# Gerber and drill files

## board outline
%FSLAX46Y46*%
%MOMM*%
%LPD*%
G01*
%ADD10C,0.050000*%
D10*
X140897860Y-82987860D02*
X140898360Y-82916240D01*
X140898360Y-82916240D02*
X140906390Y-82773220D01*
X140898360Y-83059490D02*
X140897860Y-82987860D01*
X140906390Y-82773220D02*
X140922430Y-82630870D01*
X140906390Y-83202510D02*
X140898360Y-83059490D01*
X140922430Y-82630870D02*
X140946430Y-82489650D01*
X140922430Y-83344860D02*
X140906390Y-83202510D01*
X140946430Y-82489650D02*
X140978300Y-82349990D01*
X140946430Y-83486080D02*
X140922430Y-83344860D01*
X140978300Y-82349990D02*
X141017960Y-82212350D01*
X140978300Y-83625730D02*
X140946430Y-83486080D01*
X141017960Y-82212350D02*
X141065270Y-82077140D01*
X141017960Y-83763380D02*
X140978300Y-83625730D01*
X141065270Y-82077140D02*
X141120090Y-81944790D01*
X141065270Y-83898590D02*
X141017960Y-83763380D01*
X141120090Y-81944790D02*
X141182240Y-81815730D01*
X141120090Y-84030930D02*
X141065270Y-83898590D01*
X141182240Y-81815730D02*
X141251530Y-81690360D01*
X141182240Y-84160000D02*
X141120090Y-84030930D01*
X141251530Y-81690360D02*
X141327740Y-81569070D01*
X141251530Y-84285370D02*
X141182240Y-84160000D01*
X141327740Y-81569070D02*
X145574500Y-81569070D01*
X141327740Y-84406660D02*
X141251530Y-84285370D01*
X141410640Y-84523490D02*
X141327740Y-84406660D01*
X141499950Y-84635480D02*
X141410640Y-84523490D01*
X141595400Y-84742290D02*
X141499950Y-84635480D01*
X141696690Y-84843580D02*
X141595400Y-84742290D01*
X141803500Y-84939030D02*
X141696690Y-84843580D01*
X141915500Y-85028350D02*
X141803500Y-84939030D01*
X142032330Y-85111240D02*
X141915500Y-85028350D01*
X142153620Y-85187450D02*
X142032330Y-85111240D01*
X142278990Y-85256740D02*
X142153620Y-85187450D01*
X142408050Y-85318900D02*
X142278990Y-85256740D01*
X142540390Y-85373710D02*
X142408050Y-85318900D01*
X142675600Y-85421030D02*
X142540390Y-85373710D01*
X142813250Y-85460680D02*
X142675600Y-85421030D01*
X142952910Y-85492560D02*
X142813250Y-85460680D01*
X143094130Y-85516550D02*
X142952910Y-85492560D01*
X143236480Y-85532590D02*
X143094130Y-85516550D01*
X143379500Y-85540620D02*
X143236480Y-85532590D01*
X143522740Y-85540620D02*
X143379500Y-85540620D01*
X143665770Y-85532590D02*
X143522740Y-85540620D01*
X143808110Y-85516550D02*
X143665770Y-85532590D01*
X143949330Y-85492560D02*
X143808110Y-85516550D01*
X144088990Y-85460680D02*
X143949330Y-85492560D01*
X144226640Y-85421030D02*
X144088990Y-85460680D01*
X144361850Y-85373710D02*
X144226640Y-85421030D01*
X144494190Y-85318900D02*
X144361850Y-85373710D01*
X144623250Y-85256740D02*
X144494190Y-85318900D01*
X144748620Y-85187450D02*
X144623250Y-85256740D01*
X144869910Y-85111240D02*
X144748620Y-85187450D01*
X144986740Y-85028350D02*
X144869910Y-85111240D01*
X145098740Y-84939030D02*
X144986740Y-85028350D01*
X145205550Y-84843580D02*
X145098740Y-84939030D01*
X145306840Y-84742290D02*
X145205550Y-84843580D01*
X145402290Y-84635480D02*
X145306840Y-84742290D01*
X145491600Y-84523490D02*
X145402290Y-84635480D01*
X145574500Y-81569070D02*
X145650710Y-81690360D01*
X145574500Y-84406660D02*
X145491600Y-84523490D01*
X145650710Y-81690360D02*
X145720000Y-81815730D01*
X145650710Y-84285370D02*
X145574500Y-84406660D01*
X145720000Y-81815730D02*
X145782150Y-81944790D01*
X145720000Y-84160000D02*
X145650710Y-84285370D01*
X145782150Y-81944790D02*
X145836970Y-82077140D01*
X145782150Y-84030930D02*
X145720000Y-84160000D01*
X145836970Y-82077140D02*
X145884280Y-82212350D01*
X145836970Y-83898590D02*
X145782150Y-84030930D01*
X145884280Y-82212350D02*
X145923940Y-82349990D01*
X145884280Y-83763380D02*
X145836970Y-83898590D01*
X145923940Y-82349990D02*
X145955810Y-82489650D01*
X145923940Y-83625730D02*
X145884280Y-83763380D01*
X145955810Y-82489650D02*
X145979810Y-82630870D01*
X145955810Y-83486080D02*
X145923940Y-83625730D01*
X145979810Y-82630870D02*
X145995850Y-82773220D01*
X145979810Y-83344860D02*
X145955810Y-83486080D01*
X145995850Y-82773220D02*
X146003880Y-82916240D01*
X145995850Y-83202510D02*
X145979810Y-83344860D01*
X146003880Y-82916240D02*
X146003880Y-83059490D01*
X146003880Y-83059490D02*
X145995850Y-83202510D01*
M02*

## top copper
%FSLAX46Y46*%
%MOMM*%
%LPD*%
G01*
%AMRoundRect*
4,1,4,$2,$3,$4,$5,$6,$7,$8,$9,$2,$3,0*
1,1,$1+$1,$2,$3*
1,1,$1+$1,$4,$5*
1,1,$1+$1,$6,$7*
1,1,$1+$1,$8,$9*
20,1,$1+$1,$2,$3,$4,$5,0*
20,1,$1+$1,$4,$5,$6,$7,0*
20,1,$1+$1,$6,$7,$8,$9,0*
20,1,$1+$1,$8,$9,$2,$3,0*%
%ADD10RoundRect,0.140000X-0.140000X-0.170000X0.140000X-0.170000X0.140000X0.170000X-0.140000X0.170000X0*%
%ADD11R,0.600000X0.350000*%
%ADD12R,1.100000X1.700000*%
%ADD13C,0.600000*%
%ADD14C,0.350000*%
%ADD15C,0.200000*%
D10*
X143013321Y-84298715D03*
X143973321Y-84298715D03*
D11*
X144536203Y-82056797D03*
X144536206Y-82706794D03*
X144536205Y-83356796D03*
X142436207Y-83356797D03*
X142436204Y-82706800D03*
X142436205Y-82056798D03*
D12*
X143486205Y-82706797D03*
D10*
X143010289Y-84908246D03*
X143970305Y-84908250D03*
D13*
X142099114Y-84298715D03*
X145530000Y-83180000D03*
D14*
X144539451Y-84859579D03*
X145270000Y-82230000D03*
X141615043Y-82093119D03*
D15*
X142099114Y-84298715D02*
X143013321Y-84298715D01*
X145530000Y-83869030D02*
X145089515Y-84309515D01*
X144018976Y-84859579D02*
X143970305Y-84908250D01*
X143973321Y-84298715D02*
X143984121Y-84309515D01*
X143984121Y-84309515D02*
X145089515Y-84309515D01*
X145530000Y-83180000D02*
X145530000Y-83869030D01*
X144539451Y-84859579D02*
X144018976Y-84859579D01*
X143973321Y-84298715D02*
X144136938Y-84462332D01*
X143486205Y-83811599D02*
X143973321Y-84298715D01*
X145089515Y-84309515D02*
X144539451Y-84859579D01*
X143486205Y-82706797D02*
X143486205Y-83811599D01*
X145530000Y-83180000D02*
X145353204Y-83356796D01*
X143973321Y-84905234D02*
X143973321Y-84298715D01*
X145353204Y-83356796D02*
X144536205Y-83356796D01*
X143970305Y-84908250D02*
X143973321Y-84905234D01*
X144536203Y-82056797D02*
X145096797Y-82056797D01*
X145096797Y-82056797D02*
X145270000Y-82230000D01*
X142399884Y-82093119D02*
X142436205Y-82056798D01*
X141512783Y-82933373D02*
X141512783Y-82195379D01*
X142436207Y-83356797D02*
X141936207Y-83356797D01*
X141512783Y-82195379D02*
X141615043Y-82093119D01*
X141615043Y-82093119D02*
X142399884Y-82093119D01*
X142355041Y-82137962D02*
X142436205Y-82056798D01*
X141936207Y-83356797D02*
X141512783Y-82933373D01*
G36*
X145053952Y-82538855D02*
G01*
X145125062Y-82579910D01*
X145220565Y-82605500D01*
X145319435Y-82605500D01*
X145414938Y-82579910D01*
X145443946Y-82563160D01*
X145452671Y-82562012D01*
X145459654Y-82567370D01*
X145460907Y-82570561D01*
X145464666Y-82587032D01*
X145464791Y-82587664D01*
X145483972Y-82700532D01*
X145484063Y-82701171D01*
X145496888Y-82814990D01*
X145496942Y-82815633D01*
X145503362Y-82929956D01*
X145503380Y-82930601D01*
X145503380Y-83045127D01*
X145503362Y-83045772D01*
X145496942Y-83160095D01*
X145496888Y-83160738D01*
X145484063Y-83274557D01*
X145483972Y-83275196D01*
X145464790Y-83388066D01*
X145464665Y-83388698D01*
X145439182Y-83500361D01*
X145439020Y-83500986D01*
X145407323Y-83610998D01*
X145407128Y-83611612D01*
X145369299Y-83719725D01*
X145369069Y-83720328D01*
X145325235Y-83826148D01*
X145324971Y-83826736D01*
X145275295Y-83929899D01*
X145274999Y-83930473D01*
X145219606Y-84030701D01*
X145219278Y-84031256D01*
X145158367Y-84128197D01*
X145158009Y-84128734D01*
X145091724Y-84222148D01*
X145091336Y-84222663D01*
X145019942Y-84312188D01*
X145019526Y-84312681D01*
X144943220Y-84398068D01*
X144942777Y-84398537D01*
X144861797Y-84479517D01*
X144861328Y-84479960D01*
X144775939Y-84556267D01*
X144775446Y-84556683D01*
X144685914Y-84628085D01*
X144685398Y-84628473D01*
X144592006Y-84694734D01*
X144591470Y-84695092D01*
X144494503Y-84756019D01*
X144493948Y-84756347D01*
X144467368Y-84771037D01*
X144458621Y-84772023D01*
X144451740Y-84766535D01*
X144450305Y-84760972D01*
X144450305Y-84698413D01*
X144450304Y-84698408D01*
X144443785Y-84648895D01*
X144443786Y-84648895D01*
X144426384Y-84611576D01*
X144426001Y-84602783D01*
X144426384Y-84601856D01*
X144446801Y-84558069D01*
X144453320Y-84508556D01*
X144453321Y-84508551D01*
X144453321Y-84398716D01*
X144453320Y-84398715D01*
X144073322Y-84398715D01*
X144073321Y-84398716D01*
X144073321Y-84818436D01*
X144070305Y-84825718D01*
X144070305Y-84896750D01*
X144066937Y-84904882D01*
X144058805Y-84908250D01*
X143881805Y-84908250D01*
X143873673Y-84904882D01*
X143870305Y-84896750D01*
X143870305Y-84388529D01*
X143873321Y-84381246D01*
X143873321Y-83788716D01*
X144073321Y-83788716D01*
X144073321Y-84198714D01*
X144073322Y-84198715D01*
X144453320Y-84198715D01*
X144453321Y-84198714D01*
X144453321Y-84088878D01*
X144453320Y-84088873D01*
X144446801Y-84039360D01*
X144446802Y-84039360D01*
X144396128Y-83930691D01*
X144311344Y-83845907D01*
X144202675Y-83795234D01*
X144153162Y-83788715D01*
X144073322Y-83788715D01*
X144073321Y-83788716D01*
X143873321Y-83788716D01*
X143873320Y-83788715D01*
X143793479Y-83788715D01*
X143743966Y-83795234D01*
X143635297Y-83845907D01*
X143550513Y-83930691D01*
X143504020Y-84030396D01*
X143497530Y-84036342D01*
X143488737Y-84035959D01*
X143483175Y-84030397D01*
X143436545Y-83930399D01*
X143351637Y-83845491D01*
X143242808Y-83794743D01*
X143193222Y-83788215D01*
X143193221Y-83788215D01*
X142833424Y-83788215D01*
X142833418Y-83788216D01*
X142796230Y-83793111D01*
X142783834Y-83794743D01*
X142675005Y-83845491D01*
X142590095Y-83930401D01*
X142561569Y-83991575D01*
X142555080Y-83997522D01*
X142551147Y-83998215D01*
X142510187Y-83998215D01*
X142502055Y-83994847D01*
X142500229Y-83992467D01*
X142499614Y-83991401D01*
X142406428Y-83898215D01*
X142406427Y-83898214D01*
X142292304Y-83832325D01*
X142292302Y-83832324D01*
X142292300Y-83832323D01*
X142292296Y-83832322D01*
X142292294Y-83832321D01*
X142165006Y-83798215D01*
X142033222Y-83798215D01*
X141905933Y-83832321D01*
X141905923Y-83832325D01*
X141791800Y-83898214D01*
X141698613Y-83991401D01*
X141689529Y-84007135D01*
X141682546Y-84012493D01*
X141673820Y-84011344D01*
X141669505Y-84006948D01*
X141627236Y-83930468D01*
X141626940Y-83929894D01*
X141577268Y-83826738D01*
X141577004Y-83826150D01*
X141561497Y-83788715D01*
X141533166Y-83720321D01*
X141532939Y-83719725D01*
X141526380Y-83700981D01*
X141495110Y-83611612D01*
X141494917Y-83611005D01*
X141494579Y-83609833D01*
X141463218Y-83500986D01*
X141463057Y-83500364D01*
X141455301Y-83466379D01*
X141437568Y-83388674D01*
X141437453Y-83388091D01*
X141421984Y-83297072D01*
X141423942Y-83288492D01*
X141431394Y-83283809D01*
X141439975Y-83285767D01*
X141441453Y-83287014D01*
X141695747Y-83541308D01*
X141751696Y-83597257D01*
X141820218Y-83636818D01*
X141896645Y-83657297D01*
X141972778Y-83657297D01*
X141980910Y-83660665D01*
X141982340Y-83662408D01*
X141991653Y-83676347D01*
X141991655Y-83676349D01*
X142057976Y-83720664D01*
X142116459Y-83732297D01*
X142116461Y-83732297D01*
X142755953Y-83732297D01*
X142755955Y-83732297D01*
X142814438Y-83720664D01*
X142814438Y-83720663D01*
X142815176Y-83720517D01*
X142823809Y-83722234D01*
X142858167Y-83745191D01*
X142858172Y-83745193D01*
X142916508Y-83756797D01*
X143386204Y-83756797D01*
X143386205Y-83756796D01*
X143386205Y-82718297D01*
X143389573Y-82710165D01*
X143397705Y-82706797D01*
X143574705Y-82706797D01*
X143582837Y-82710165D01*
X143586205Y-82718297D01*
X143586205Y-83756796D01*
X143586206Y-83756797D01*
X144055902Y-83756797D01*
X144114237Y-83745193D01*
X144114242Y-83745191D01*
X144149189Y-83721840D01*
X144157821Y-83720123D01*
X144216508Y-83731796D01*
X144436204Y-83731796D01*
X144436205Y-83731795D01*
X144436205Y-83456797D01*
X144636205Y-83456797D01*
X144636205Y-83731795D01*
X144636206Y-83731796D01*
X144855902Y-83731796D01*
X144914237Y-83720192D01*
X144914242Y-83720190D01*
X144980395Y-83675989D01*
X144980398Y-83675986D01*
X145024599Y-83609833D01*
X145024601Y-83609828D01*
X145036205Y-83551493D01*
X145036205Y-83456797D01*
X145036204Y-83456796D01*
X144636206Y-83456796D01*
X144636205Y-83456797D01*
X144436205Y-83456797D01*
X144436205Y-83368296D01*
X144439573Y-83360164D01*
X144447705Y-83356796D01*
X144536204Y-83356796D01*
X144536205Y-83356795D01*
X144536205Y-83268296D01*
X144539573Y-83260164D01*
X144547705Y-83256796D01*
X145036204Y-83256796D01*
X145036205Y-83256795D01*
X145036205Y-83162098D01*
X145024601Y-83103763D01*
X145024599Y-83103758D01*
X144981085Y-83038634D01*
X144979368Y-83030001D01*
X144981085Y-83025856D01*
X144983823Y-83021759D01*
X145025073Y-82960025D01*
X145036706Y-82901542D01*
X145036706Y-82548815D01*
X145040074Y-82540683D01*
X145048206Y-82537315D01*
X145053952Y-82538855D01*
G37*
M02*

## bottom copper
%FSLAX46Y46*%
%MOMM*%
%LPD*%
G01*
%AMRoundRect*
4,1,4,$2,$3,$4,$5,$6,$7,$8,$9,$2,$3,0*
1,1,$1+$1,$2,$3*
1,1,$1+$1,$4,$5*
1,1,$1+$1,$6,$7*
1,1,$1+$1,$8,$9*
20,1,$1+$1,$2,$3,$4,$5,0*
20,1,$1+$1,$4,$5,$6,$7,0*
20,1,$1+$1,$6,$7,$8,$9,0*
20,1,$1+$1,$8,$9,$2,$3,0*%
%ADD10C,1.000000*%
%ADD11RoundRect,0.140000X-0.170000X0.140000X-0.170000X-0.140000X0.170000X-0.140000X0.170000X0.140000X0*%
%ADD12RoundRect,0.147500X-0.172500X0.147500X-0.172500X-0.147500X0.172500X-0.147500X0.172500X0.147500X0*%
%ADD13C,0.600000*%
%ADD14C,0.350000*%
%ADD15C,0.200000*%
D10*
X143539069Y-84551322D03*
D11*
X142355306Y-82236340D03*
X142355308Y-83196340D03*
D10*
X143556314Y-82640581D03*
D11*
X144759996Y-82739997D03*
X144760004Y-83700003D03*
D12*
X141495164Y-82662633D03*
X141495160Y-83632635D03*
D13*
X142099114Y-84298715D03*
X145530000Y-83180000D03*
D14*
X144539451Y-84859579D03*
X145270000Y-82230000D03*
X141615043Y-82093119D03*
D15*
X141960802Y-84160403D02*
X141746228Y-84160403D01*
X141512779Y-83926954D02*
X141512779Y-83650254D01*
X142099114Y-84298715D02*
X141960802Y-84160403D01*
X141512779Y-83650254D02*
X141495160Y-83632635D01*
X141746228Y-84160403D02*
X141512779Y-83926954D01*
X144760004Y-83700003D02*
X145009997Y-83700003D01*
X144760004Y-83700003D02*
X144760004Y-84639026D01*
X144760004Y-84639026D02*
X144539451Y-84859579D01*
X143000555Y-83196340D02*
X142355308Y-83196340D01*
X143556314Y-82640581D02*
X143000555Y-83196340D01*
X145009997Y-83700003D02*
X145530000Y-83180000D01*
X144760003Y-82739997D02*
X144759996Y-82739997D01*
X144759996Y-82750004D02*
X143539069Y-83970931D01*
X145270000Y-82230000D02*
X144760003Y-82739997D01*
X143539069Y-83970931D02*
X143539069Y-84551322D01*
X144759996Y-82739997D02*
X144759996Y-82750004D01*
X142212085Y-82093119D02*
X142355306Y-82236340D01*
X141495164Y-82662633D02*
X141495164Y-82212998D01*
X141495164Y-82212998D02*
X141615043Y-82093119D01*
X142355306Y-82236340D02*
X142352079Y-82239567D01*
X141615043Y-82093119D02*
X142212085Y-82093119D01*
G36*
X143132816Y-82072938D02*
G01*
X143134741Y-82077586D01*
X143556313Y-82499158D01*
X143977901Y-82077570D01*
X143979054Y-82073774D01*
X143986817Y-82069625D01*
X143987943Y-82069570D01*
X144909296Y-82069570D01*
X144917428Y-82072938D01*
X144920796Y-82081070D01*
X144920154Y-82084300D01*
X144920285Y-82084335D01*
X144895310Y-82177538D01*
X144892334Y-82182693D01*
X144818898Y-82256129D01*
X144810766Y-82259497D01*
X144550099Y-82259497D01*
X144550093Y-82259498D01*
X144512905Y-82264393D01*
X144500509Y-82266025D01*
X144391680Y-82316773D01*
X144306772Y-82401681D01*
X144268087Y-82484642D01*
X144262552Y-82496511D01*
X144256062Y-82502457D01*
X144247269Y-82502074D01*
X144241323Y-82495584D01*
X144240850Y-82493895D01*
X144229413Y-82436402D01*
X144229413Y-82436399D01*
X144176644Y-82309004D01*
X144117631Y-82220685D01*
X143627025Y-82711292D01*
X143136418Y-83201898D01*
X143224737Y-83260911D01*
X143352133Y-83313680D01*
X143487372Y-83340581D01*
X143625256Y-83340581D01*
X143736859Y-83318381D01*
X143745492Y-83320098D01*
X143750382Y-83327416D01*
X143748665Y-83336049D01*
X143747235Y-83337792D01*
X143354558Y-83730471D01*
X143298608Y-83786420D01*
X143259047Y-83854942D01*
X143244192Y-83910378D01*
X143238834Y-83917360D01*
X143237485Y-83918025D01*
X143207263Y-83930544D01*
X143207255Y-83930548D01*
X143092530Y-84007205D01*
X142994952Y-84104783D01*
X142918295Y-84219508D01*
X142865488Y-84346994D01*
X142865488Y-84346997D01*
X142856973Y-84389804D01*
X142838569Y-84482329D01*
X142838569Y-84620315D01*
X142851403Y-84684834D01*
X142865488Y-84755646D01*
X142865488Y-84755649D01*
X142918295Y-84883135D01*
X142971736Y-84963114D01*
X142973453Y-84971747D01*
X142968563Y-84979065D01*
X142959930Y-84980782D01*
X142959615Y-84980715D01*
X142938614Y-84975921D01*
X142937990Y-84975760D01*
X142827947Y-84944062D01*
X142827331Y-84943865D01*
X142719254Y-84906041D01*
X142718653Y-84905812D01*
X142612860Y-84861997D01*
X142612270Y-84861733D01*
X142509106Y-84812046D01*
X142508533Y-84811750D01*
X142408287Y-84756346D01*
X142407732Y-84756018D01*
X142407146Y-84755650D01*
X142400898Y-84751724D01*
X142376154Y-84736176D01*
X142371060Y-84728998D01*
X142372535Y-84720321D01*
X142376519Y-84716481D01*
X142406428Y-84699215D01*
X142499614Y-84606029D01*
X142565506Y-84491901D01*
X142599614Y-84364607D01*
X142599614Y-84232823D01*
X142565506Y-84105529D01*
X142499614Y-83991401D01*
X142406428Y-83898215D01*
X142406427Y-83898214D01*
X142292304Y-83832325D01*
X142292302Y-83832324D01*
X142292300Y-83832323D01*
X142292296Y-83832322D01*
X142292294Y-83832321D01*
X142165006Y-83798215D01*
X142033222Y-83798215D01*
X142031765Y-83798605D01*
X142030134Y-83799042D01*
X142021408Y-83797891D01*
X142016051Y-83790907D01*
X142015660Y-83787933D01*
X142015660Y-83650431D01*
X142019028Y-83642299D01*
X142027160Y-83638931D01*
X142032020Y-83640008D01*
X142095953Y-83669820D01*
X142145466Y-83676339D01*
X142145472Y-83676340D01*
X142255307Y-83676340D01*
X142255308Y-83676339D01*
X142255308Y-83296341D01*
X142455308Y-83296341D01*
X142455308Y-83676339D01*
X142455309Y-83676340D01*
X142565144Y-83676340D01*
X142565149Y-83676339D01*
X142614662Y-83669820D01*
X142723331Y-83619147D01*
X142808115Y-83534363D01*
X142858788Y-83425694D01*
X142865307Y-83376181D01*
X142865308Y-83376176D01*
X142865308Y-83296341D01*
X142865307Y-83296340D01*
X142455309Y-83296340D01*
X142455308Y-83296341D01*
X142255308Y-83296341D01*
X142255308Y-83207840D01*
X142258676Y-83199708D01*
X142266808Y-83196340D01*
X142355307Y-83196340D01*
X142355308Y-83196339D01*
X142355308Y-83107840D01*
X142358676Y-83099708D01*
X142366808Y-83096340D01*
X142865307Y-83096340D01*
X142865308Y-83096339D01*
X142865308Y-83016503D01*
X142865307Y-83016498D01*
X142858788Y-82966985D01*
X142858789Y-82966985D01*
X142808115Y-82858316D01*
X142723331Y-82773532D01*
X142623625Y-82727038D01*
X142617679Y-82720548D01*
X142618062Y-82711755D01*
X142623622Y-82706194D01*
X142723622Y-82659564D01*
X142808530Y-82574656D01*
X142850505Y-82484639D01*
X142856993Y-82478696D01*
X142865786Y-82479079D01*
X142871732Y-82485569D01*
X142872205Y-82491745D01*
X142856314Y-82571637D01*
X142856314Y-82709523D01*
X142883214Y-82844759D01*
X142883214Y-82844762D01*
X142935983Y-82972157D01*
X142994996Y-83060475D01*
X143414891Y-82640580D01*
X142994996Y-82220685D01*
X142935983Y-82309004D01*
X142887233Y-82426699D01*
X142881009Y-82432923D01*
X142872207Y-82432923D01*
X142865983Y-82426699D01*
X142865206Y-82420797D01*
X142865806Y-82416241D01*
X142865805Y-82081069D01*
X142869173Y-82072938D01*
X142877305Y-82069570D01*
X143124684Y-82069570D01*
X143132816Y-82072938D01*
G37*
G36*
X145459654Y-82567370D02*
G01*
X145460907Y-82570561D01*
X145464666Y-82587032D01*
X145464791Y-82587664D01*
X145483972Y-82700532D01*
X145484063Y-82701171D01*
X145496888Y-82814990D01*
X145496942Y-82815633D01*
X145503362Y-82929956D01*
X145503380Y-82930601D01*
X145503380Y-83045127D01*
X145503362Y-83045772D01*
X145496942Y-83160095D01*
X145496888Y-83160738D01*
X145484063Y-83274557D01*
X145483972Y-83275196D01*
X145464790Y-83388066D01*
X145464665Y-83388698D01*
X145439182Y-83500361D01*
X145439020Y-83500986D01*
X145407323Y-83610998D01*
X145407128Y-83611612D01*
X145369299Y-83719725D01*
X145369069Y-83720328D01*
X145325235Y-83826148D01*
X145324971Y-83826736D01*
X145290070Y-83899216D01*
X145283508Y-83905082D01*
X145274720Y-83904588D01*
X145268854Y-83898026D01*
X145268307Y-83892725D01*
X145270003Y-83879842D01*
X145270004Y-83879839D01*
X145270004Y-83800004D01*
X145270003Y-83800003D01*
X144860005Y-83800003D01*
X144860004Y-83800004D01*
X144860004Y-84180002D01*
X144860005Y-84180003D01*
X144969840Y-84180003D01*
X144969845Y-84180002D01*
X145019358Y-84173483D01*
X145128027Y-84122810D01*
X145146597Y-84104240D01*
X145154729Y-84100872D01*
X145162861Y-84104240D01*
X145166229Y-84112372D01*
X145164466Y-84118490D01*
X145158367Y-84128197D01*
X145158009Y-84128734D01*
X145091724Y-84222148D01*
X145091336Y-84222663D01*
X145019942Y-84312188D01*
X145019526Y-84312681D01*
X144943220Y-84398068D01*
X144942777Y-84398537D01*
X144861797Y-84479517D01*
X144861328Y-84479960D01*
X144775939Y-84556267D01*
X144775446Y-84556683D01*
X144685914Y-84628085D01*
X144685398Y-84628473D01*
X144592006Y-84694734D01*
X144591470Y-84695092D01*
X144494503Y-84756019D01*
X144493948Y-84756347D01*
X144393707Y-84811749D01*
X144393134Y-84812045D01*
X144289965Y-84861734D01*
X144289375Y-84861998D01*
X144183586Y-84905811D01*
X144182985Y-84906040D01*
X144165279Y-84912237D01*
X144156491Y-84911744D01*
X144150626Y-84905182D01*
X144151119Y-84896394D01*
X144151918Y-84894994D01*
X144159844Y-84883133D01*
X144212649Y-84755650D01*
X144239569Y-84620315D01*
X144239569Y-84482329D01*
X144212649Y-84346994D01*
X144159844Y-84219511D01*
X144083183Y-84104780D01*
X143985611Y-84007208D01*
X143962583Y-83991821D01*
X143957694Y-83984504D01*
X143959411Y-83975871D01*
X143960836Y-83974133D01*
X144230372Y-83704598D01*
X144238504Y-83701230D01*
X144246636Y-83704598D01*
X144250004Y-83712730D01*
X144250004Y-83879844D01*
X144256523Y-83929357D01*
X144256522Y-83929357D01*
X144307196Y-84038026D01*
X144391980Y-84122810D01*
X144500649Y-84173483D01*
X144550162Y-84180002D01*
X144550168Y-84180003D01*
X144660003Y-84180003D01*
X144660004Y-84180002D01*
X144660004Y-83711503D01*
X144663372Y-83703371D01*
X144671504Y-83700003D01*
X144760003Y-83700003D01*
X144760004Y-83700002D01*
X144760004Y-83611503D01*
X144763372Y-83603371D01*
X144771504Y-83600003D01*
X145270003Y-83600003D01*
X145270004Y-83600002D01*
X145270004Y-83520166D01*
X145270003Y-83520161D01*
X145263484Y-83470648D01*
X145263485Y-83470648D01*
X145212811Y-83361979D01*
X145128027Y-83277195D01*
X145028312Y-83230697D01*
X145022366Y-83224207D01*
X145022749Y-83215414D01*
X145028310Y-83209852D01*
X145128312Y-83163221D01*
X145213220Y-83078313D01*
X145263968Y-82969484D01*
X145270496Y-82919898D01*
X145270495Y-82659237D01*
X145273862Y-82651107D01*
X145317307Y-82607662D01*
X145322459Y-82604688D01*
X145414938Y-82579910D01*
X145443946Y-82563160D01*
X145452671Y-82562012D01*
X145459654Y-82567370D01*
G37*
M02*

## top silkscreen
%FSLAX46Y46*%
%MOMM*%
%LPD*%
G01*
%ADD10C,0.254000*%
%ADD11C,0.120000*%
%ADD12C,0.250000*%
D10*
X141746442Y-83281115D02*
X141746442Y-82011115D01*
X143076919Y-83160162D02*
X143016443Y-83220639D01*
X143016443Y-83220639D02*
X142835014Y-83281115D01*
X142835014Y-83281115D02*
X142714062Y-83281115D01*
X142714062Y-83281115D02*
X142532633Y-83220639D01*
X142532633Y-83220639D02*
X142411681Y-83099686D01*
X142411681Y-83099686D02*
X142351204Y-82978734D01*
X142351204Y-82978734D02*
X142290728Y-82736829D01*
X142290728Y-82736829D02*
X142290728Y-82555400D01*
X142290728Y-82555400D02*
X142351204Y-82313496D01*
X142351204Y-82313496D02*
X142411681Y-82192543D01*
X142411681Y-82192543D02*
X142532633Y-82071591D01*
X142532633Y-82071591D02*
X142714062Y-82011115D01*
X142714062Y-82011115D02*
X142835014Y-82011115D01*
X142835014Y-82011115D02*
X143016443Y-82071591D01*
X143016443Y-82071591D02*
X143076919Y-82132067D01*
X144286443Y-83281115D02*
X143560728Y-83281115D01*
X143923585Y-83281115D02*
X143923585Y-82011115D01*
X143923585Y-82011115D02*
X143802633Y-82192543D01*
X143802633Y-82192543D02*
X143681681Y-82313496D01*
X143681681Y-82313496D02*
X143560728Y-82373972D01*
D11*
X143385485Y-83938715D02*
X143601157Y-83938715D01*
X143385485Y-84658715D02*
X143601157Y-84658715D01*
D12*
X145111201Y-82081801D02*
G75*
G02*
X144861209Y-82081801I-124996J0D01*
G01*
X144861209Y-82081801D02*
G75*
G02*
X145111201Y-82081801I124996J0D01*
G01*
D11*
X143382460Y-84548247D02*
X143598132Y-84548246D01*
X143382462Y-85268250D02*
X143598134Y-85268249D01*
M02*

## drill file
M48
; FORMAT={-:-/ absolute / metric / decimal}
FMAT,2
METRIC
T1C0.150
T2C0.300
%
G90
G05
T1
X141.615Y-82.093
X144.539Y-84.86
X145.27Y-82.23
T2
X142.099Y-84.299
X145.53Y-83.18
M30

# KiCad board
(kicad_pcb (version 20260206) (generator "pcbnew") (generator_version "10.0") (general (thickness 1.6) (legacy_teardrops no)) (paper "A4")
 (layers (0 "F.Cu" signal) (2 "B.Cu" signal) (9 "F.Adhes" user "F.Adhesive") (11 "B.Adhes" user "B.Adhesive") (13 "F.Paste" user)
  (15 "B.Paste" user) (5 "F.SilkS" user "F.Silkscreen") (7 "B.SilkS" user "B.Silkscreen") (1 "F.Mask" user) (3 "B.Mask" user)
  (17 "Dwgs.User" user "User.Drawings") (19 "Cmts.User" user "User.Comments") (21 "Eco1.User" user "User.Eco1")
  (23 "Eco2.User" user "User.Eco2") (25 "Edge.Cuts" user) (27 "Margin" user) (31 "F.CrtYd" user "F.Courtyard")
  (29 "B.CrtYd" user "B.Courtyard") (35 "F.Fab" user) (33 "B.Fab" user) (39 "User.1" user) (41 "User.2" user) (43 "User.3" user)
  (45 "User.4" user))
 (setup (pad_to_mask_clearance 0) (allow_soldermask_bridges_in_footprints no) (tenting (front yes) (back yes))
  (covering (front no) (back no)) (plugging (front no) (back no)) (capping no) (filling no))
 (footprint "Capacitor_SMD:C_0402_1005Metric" (layer "F.Cu") (at 143.493321 84.298715)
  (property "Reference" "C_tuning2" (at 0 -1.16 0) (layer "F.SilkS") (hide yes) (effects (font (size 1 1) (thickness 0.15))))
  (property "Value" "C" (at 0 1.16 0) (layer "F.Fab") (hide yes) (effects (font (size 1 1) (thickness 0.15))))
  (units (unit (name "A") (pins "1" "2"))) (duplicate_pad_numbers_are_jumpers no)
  (fp_line (start -0.107836 -0.36) (end 0.107836 -0.36) (stroke (width 0.12) (type solid)) (layer "F.SilkS"))
  (fp_line (start -0.107836 0.36) (end 0.107836 0.36) (stroke (width 0.12) (type solid)) (layer "F.SilkS"))
  (pad "1" smd roundrect (at -0.48 0) (size 0.56 0.62) (layers "F.Cu" "F.Mask" "F.Paste") (roundrect_rratio 0.25) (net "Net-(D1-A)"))
  (pad "2" smd roundrect (at 0.48 0) (size 0.56 0.62) (layers "F.Cu" "F.Mask" "F.Paste") (roundrect_rratio 0.25) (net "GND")))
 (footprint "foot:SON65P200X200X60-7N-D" (layer "F.Cu") (at 143.486205 82.706797 180)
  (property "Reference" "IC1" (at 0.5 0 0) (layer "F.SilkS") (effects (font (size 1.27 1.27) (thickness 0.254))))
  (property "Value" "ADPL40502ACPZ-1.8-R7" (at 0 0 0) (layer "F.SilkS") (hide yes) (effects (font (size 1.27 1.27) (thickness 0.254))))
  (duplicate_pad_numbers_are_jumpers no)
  (fp_circle (center -1.5 0.624996) (end -1.5 0.749992) (stroke (width 0.25) (type solid)) (fill no) (layer "F.SilkS"))
  (pad "1" smd rect (at -1.049998 0.65 270) (size 0.35 0.6) (layers "F.Cu" "F.Mask" "F.Paste") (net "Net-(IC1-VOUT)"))
  (pad "2" smd rect (at -1.050001 0.000003 270) (size 0.35 0.6) (layers "F.Cu" "F.Mask" "F.Paste") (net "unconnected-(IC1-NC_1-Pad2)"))
  (pad "3" smd rect (at -1.05 -0.649999 270) (size 0.35 0.6) (layers "F.Cu" "F.Mask" "F.Paste") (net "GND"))
  (pad "4" smd rect (at 1.049998 -0.65 270) (size 0.35 0.6) (layers "F.Cu" "F.Mask" "F.Paste") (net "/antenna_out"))
  (pad "5" smd rect (at 1.050001 -0.000003 270) (size 0.35 0.6) (layers "F.Cu" "F.Mask" "F.Paste") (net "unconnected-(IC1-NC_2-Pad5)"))
  (pad "6" smd rect (at 1.05 0.649999 270) (size 0.35 0.6) (layers "F.Cu" "F.Mask" "F.Paste") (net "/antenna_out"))
  (pad "7" smd rect (at 0 0 180) (size 1.1 1.7) (layers "F.Cu" "F.Mask" "F.Paste") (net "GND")))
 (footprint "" (layer "F.Cu") (at 143.539069 84.551322)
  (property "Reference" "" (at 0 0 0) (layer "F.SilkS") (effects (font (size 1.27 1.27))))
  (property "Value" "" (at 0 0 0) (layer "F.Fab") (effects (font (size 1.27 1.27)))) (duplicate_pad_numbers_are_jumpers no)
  (pad "1" smd circle (at 0 0 180) (size 1 1) (layers "B.Cu" "B.Mask") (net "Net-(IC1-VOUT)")))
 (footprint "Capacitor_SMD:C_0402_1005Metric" (layer "F.Cu") (at 143.490297 84.908248)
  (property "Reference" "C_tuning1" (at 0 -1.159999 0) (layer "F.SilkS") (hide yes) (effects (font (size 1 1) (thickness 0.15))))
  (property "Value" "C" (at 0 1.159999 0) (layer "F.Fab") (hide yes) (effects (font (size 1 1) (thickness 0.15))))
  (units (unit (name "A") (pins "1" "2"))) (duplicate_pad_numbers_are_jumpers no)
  (fp_line (start -0.107837 -0.360001) (end 0.107835 -0.360002) (stroke (width 0.12) (type solid)) (layer "F.SilkS"))
  (fp_line (start -0.107835 0.360002) (end 0.107837 0.360001) (stroke (width 0.12) (type solid)) (layer "F.SilkS"))
  (pad "1" smd roundrect (at -0.480008 -0.000002) (size 0.56 0.62) (layers "F.Cu" "F.Mask" "F.Paste") (roundrect_rratio 0.25)
   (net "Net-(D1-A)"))
  (pad "2" smd roundrect (at 0.480008 0.000002) (size 0.56 0.62) (layers "F.Cu" "F.Mask" "F.Paste") (roundrect_rratio 0.25) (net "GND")))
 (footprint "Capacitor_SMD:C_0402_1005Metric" (layer "B.Cu") (at 142.355307 82.71634 -90)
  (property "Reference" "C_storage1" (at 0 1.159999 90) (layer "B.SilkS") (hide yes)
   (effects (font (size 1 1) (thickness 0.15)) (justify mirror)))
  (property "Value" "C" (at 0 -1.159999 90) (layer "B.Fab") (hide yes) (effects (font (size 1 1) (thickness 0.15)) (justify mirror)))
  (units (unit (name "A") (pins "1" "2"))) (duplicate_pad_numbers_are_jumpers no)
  (pad "1" smd roundrect (at -0.48 0.000001 270) (size 0.56 0.62) (layers "B.Cu" "B.Mask" "B.Paste") (roundrect_rratio 0.25)
   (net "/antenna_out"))
  (pad "2" smd roundrect (at 0.48 -0.000001 270) (size 0.56 0.62) (layers "B.Cu" "B.Mask" "B.Paste") (roundrect_rratio 0.25) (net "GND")))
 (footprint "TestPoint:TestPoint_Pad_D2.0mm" (layer "B.Cu") (at 143.556314 82.640581 180)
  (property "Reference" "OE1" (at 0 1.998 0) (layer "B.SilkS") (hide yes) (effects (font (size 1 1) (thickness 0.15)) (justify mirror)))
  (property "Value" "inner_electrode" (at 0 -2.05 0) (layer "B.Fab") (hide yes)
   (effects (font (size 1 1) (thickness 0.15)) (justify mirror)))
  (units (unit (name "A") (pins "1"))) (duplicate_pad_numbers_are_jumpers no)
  (pad "1" smd circle (at 0 0 180) (size 1 1) (layers "B.Cu" "B.Mask") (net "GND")))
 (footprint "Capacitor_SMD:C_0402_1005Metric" (layer "B.Cu") (at 144.76 83.22 -90)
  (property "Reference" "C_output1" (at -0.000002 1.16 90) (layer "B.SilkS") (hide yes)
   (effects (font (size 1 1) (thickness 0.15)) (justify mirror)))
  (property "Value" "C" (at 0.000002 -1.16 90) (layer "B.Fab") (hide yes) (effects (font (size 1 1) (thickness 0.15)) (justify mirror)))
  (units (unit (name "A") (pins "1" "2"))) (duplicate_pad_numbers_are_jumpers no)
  (pad "1" smd roundrect (at -0.480003 0.000004 270) (size 0.56 0.62) (layers "B.Cu" "B.Mask" "B.Paste") (roundrect_rratio 0.25)
   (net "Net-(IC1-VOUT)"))
  (pad "2" smd roundrect (at 0.480003 -0.000004 270) (size 0.56 0.62) (layers "B.Cu" "B.Mask" "B.Paste") (roundrect_rratio 0.25) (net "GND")))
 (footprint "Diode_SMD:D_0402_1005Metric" (layer "B.Cu") (at 141.495162 83.147634 -90)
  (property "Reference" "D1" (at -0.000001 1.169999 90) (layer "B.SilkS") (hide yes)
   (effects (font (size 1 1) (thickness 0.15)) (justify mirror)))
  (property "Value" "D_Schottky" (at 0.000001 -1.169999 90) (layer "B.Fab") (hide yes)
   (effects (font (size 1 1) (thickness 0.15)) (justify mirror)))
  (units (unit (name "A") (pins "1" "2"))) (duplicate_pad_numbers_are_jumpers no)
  (pad "1" smd roundrect (at -0.485001 -0.000002 270) (size 0.59 0.64) (layers "B.Cu" "B.Mask" "B.Paste") (roundrect_rratio 0.25)
   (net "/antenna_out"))
  (pad "2" smd roundrect (at 0.485001 0.000002 270) (size 0.59 0.64) (layers "B.Cu" "B.Mask" "B.Paste") (roundrect_rratio 0.25)
   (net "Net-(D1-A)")))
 (gr_line (start 140.89786 82.98786) (end 140.89836 82.91624) (stroke (width 0.05) (type solid)) (layer "Edge.Cuts"))
 (gr_line (start 140.89836 82.91624) (end 140.90639 82.77322) (stroke (width 0.05) (type solid)) (layer "Edge.Cuts"))
 (gr_line (start 140.89836 83.05949) (end 140.89786 82.98786) (stroke (width 0.05) (type solid)) (layer "Edge.Cuts"))
 (gr_line (start 140.90639 82.77322) (end 140.92243 82.63087) (stroke (width 0.05) (type solid)) (layer "Edge.Cuts"))
 (gr_line (start 140.90639 83.20251) (end 140.89836 83.05949) (stroke (width 0.05) (type solid)) (layer "Edge.Cuts"))
 (gr_line (start 140.92243 82.63087) (end 140.94643 82.48965) (stroke (width 0.05) (type solid)) (layer "Edge.Cuts"))
 (gr_line (start 140.92243 83.34486) (end 140.90639 83.20251) (stroke (width 0.05) (type solid)) (layer "Edge.Cuts"))
 (gr_line (start 140.94643 82.48965) (end 140.9783 82.34999) (stroke (width 0.05) (type solid)) (layer "Edge.Cuts"))
 (gr_line (start 140.94643 83.48608) (end 140.92243 83.34486) (stroke (width 0.05) (type solid)) (layer "Edge.Cuts"))
 (gr_line (start 140.9783 82.34999) (end 141.01796 82.21235) (stroke (width 0.05) (type solid)) (layer "Edge.Cuts"))
 (gr_line (start 140.9783 83.62573) (end 140.94643 83.48608) (stroke (width 0.05) (type solid)) (layer "Edge.Cuts"))
 (gr_line (start 141.01796 82.21235) (end 141.06527 82.07714) (stroke (width 0.05) (type solid)) (layer "Edge.Cuts"))
 (gr_line (start 141.01796 83.76338) (end 140.9783 83.62573) (stroke (width 0.05) (type solid)) (layer "Edge.Cuts"))
 (gr_line (start 141.06527 82.07714) (end 141.12009 81.94479) (stroke (width 0.05) (type solid)) (layer "Edge.Cuts"))
 (gr_line (start 141.06527 83.89859) (end 141.01796 83.76338) (stroke (width 0.05) (type solid)) (layer "Edge.Cuts"))
 (gr_line (start 141.12009 81.94479) (end 141.18224 81.81573) (stroke (width 0.05) (type solid)) (layer "Edge.Cuts"))
 (gr_line (start 141.12009 84.03093) (end 141.06527 83.89859) (stroke (width 0.05) (type solid)) (layer "Edge.Cuts"))
 (gr_line (start 141.18224 81.81573) (end 141.25153 81.69036) (stroke (width 0.05) (type solid)) (layer "Edge.Cuts"))
 (gr_line (start 141.18224 84.16) (end 141.12009 84.03093) (stroke (width 0.05) (type solid)) (layer "Edge.Cuts"))
 (gr_line (start 141.25153 81.69036) (end 141.32774 81.56907) (stroke (width 0.05) (type solid)) (layer "Edge.Cuts"))
 (gr_line (start 141.25153 84.28537) (end 141.18224 84.16) (stroke (width 0.05) (type solid)) (layer "Edge.Cuts"))
 (gr_line (start 141.32774 81.56907) (end 145.5745 81.56907) (stroke (width 0.05) (type solid)) (layer "Edge.Cuts"))
 (gr_line (start 141.32774 84.40666) (end 141.25153 84.28537) (stroke (width 0.05) (type solid)) (layer "Edge.Cuts"))
 (gr_line (start 141.41064 84.52349) (end 141.32774 84.40666) (stroke (width 0.05) (type solid)) (layer "Edge.Cuts"))
 (gr_line (start 141.49995 84.63548) (end 141.41064 84.52349) (stroke (width 0.05) (type solid)) (layer "Edge.Cuts"))
 (gr_line (start 141.5954 84.74229) (end 141.49995 84.63548) (stroke (width 0.05) (type solid)) (layer "Edge.Cuts"))
 (gr_line (start 141.69669 84.84358) (end 141.5954 84.74229) (stroke (width 0.05) (type solid)) (layer "Edge.Cuts"))
 (gr_line (start 141.8035 84.93903) (end 141.69669 84.84358) (stroke (width 0.05) (type solid)) (layer "Edge.Cuts"))
 (gr_line (start 141.9155 85.02835) (end 141.8035 84.93903) (stroke (width 0.05) (type solid)) (layer "Edge.Cuts"))
 (gr_line (start 142.03233 85.11124) (end 141.9155 85.02835) (stroke (width 0.05) (type solid)) (layer "Edge.Cuts"))
 (gr_line (start 142.15362 85.18745) (end 142.03233 85.11124) (stroke (width 0.05) (type solid)) (layer "Edge.Cuts"))
 (gr_line (start 142.27899 85.25674) (end 142.15362 85.18745) (stroke (width 0.05) (type solid)) (layer "Edge.Cuts"))
 (gr_line (start 142.40805 85.3189) (end 142.27899 85.25674) (stroke (width 0.05) (type solid)) (layer "Edge.Cuts"))
 (gr_line (start 142.54039 85.37371) (end 142.40805 85.3189) (stroke (width 0.05) (type solid)) (layer "Edge.Cuts"))
 (gr_line (start 142.6756 85.42103) (end 142.54039 85.37371) (stroke (width 0.05) (type solid)) (layer "Edge.Cuts"))
 (gr_line (start 142.81325 85.46068) (end 142.6756 85.42103) (stroke (width 0.05) (type solid)) (layer "Edge.Cuts"))
 (gr_line (start 142.95291 85.49256) (end 142.81325 85.46068) (stroke (width 0.05) (type solid)) (layer "Edge.Cuts"))
 (gr_line (start 143.09413 85.51655) (end 142.95291 85.49256) (stroke (width 0.05) (type solid)) (layer "Edge.Cuts"))
 (gr_line (start 143.23648 85.53259) (end 143.09413 85.51655) (stroke (width 0.05) (type solid)) (layer "Edge.Cuts"))
 (gr_line (start 143.3795 85.54062) (end 143.23648 85.53259) (stroke (width 0.05) (type solid)) (layer "Edge.Cuts"))
 (gr_line (start 143.52274 85.54062) (end 143.3795 85.54062) (stroke (width 0.05) (type solid)) (layer "Edge.Cuts"))
 (gr_line (start 143.66577 85.53259) (end 143.52274 85.54062) (stroke (width 0.05) (type solid)) (layer "Edge.Cuts"))
 (gr_line (start 143.80811 85.51655) (end 143.66577 85.53259) (stroke (width 0.05) (type solid)) (layer "Edge.Cuts"))
 (gr_line (start 143.94933 85.49256) (end 143.80811 85.51655) (stroke (width 0.05) (type solid)) (layer "Edge.Cuts"))
 (gr_line (start 144.08899 85.46068) (end 143.94933 85.49256) (stroke (width 0.05) (type solid)) (layer "Edge.Cuts"))
 (gr_line (start 144.22664 85.42103) (end 144.08899 85.46068) (stroke (width 0.05) (type solid)) (layer "Edge.Cuts"))
 (gr_line (start 144.36185 85.37371) (end 144.22664 85.42103) (stroke (width 0.05) (type solid)) (layer "Edge.Cuts"))
 (gr_line (start 144.49419 85.3189) (end 144.36185 85.37371) (stroke (width 0.05) (type solid)) (layer "Edge.Cuts"))
 (gr_line (start 144.62325 85.25674) (end 144.49419 85.3189) (stroke (width 0.05) (type solid)) (layer "Edge.Cuts"))
 (gr_line (start 144.74862 85.18745) (end 144.62325 85.25674) (stroke (width 0.05) (type solid)) (layer "Edge.Cuts"))
 (gr_line (start 144.86991 85.11124) (end 144.74862 85.18745) (stroke (width 0.05) (type solid)) (layer "Edge.Cuts"))
 (gr_line (start 144.98674 85.02835) (end 144.86991 85.11124) (stroke (width 0.05) (type solid)) (layer "Edge.Cuts"))
 (gr_line (start 145.09874 84.93903) (end 144.98674 85.02835) (stroke (width 0.05) (type solid)) (layer "Edge.Cuts"))
 (gr_line (start 145.20555 84.84358) (end 145.09874 84.93903) (stroke (width 0.05) (type solid)) (layer "Edge.Cuts"))
 (gr_line (start 145.30684 84.74229) (end 145.20555 84.84358) (stroke (width 0.05) (type solid)) (layer "Edge.Cuts"))
 (gr_line (start 145.40229 84.63548) (end 145.30684 84.74229) (stroke (width 0.05) (type solid)) (layer "Edge.Cuts"))
 (gr_line (start 145.4916 84.52349) (end 145.40229 84.63548) (stroke (width 0.05) (type solid)) (layer "Edge.Cuts"))
 (gr_line (start 145.5745 81.56907) (end 145.65071 81.69036) (stroke (width 0.05) (type solid)) (layer "Edge.Cuts"))
 (gr_line (start 145.5745 84.40666) (end 145.4916 84.52349) (stroke (width 0.05) (type solid)) (layer "Edge.Cuts"))
 (gr_line (start 145.65071 81.69036) (end 145.72 81.81573) (stroke (width 0.05) (type solid)) (layer "Edge.Cuts"))
 (gr_line (start 145.65071 84.28537) (end 145.5745 84.40666) (stroke (width 0.05) (type solid)) (layer "Edge.Cuts"))
 (gr_line (start 145.72 81.81573) (end 145.78215 81.94479) (stroke (width 0.05) (type solid)) (layer "Edge.Cuts"))
 (gr_line (start 145.72 84.16) (end 145.65071 84.28537) (stroke (width 0.05) (type solid)) (layer "Edge.Cuts"))
 (gr_line (start 145.78215 81.94479) (end 145.83697 82.07714) (stroke (width 0.05) (type solid)) (layer "Edge.Cuts"))
 (gr_line (start 145.78215 84.03093) (end 145.72 84.16) (stroke (width 0.05) (type solid)) (layer "Edge.Cuts"))
 (gr_line (start 145.83697 82.07714) (end 145.88428 82.21235) (stroke (width 0.05) (type solid)) (layer "Edge.Cuts"))
 (gr_line (start 145.83697 83.89859) (end 145.78215 84.03093) (stroke (width 0.05) (type solid)) (layer "Edge.Cuts"))
 (gr_line (start 145.88428 82.21235) (end 145.92394 82.34999) (stroke (width 0.05) (type solid)) (layer "Edge.Cuts"))
 (gr_line (start 145.88428 83.76338) (end 145.83697 83.89859) (stroke (width 0.05) (type solid)) (layer "Edge.Cuts"))
 (gr_line (start 145.92394 82.34999) (end 145.95581 82.48965) (stroke (width 0.05) (type solid)) (layer "Edge.Cuts"))
 (gr_line (start 145.92394 83.62573) (end 145.88428 83.76338) (stroke (width 0.05) (type solid)) (layer "Edge.Cuts"))
 (gr_line (start 145.95581 82.48965) (end 145.97981 82.63087) (stroke (width 0.05) (type solid)) (layer "Edge.Cuts"))
 (gr_line (start 145.95581 83.48608) (end 145.92394 83.62573) (stroke (width 0.05) (type solid)) (layer "Edge.Cuts"))
 (gr_line (start 145.97981 82.63087) (end 145.99585 82.77322) (stroke (width 0.05) (type solid)) (layer "Edge.Cuts"))
 (gr_line (start 145.97981 83.34486) (end 145.95581 83.48608) (stroke (width 0.05) (type solid)) (layer "Edge.Cuts"))
 (gr_line (start 145.99585 82.77322) (end 146.00388 82.91624) (stroke (width 0.05) (type solid)) (layer "Edge.Cuts"))
 (gr_line (start 145.99585 83.20251) (end 145.97981 83.34486) (stroke (width 0.05) (type solid)) (layer "Edge.Cuts"))
 (gr_line (start 146.00388 82.91624) (end 146.00388 83.05949) (stroke (width 0.05) (type solid)) (layer "Edge.Cuts"))
 (gr_line (start 146.00388 83.05949) (end 145.99585 83.20251) (stroke (width 0.05) (type solid)) (layer "Edge.Cuts"))
 (segment (start 142.099114 84.298715) (end 143.013321 84.298715) (width 0.2) (layer "F.Cu") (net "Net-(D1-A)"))
 (via (at 142.099114 84.298715) (size 0.6) (drill 0.3) (layers "F.Cu" "B.Cu") (free yes) (tenting (front no) (back no)) (capping no)
  (covering (front no) (back no)) (plugging (front no) (back no)) (filling no) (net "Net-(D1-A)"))
 (segment (start 141.960802 84.160403) (end 141.746228 84.160403) (width 0.2) (layer "B.Cu") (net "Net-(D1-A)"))
 (segment (start 141.512779 83.926954) (end 141.512779 83.650254) (width 0.2) (layer "B.Cu") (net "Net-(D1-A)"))
 (segment (start 142.099114 84.298715) (end 141.960802 84.160403) (width 0.2) (layer "B.Cu") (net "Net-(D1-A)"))
 (segment (start 141.512779 83.650254) (end 141.49516 83.632635) (width 0.2) (layer "B.Cu") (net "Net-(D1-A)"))
 (segment (start 141.746228 84.160403) (end 141.512779 83.926954) (width 0.2) (layer "B.Cu") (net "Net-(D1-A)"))
 (segment (start 145.53 83.86903) (end 145.089515 84.309515) (width 0.2) (layer "F.Cu") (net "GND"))
 (segment (start 144.018976 84.859579) (end 143.970305 84.90825) (width 0.2) (layer "F.Cu") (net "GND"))
 (segment (start 143.973321 84.298715) (end 143.984121 84.309515) (width 0.2) (layer "F.Cu") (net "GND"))
 (segment (start 143.984121 84.309515) (end 145.089515 84.309515) (width 0.2) (layer "F.Cu") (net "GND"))
 (segment (start 145.53 83.18) (end 145.53 83.86903) (width 0.2) (layer "F.Cu") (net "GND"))
 (segment (start 144.539451 84.859579) (end 144.018976 84.859579) (width 0.2) (layer "F.Cu") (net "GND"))
 (segment (start 143.973321 84.298715) (end 144.136938 84.462332) (width 0.2) (layer "F.Cu") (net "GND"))
 (segment (start 143.486205 83.811599) (end 143.973321 84.298715) (width 0.2) (layer "F.Cu") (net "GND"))
 (segment (start 145.089515 84.309515) (end 144.539451 84.859579) (width 0.2) (layer "F.Cu") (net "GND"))
 (segment (start 143.486205 82.706797) (end 143.486205 83.811599) (width 0.2) (layer "F.Cu") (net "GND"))
 (segment (start 145.53 83.18) (end 145.353204 83.356796) (width 0.2) (layer "F.Cu") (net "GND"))
 (segment (start 143.973321 84.905234) (end 143.973321 84.298715) (width 0.2) (layer "F.Cu") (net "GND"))
 (segment (start 145.353204 83.356796) (end 144.536205 83.356796) (width 0.2) (layer "F.Cu") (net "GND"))
 (segment (start 143.970305 84.90825) (end 143.973321 84.905234) (width 0.2) (layer "F.Cu") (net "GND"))
 (via (at 145.53 83.18) (size 0.6) (drill 0.3) (layers "F.Cu" "B.Cu") (free yes) (tenting (front no) (back no)) (capping no)
  (covering (front no) (back no)) (plugging (front no) (back no)) (filling no) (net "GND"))
 (via (at 144.539451 84.859579) (size 0.35) (drill 0.15) (layers "F.Cu" "B.Cu") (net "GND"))
 (segment (start 144.760004 83.700003) (end 145.009997 83.700003) (width 0.2) (layer "B.Cu") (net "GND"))
 (segment (start 144.760004 83.700003) (end 144.760004 84.639026) (width 0.2) (layer "B.Cu") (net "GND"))
 (segment (start 144.760004 84.639026) (end 144.539451 84.859579) (width 0.2) (layer "B.Cu") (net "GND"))
 (segment (start 143.000555 83.19634) (end 142.355308 83.19634) (width 0.2) (layer "B.Cu") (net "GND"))
 (segment (start 143.556314 82.640581) (end 143.000555 83.19634) (width 0.2) (layer "B.Cu") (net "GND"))
 (segment (start 145.009997 83.700003) (end 145.53 83.18) (width 0.2) (layer "B.Cu") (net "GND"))
 (segment (start 144.536203 82.056797) (end 145.096797 82.056797) (width 0.2) (layer "F.Cu") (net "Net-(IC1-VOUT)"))
 (segment (start 145.096797 82.056797) (end 145.27 82.23) (width 0.2) (layer "F.Cu") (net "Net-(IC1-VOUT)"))
 (via (at 145.27 82.23) (size 0.35) (drill 0.15) (layers "F.Cu" "B.Cu") (free yes) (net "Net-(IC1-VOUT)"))
 (segment (start 144.760003 82.739997) (end 144.759996 82.739997) (width 0.2) (layer "B.Cu") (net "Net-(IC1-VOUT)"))
 (segment (start 144.759996 82.750004) (end 143.539069 83.970931) (width 0.2) (layer "B.Cu") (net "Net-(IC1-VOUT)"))
 (segment (start 145.27 82.23) (end 144.760003 82.739997) (width 0.2) (layer "B.Cu") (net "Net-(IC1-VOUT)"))
 (segment (start 143.539069 83.970931) (end 143.539069 84.551322) (width 0.2) (layer "B.Cu") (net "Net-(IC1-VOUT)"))
 (segment (start 144.759996 82.739997) (end 144.759996 82.750004) (width 0.2) (layer "B.Cu") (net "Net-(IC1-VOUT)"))
 (segment (start 142.399884 82.093119) (end 142.436205 82.056798) (width 0.2) (layer "F.Cu") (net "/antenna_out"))
 (segment (start 141.512783 82.933373) (end 141.512783 82.195379) (width 0.2) (layer "F.Cu") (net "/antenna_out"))
 (segment (start 142.436207 83.356797) (end 141.936207 83.356797) (width 0.2) (layer "F.Cu") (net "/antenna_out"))
 (segment (start 141.512783 82.195379) (end 141.615043 82.093119) (width 0.2) (layer "F.Cu") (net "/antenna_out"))
 (segment (start 141.615043 82.093119) (end 142.399884 82.093119) (width 0.2) (layer "F.Cu") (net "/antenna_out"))
 (segment (start 142.355041 82.137962) (end 142.436205 82.056798) (width 0.2) (layer "F.Cu") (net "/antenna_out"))
 (segment (start 141.936207 83.356797) (end 141.512783 82.933373) (width 0.2) (layer "F.Cu") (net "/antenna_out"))
 (via (at 141.615043 82.093119) (size 0.35) (drill 0.15) (layers "F.Cu" "B.Cu") (free yes) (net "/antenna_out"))
 (segment (start 142.212085 82.093119) (end 142.355306 82.23634) (width 0.2) (layer "B.Cu") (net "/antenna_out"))
 (segment (start 141.495164 82.662633) (end 141.495164 82.212998) (width 0.2) (layer "B.Cu") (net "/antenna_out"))
 (segment (start 141.495164 82.212998) (end 141.615043 82.093119) (width 0.2) (layer "B.Cu") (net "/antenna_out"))
 (segment (start 142.355306 82.23634) (end 142.352079 82.239567) (width 0.2) (layer "B.Cu") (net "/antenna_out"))
 (segment (start 141.615043 82.093119) (end 142.212085 82.093119) (width 0.2) (layer "B.Cu") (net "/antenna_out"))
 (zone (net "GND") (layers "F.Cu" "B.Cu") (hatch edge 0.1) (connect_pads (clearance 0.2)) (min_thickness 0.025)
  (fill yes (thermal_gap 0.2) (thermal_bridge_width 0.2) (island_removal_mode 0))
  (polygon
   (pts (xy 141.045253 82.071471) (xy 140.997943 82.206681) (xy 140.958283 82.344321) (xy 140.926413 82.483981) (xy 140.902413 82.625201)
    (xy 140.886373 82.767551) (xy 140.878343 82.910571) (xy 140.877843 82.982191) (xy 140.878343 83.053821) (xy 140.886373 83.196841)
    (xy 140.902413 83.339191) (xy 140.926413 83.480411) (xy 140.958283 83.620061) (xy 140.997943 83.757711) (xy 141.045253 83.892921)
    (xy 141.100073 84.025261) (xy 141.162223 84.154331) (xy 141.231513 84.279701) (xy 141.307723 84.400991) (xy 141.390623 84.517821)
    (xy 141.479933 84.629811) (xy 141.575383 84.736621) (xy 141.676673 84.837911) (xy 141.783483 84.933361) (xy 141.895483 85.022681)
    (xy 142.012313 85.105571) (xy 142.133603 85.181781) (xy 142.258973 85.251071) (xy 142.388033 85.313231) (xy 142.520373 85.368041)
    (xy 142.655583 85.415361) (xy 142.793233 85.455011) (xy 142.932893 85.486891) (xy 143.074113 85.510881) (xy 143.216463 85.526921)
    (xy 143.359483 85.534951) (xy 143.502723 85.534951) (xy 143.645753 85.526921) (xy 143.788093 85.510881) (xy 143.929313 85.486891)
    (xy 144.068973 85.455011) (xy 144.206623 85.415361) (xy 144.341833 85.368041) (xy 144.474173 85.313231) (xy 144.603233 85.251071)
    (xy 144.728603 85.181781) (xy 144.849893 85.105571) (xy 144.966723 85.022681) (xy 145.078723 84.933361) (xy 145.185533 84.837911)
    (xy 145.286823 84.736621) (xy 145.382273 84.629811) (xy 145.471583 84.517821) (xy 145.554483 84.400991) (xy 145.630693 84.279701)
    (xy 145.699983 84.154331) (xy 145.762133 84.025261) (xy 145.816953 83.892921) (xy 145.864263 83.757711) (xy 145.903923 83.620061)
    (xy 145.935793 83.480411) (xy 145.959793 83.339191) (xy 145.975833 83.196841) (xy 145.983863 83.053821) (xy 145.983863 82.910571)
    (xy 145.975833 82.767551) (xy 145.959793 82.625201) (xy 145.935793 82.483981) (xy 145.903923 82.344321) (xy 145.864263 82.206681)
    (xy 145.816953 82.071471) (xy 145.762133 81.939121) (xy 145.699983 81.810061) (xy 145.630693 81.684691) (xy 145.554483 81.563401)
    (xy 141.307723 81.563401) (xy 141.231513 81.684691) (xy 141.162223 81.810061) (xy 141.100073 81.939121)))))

